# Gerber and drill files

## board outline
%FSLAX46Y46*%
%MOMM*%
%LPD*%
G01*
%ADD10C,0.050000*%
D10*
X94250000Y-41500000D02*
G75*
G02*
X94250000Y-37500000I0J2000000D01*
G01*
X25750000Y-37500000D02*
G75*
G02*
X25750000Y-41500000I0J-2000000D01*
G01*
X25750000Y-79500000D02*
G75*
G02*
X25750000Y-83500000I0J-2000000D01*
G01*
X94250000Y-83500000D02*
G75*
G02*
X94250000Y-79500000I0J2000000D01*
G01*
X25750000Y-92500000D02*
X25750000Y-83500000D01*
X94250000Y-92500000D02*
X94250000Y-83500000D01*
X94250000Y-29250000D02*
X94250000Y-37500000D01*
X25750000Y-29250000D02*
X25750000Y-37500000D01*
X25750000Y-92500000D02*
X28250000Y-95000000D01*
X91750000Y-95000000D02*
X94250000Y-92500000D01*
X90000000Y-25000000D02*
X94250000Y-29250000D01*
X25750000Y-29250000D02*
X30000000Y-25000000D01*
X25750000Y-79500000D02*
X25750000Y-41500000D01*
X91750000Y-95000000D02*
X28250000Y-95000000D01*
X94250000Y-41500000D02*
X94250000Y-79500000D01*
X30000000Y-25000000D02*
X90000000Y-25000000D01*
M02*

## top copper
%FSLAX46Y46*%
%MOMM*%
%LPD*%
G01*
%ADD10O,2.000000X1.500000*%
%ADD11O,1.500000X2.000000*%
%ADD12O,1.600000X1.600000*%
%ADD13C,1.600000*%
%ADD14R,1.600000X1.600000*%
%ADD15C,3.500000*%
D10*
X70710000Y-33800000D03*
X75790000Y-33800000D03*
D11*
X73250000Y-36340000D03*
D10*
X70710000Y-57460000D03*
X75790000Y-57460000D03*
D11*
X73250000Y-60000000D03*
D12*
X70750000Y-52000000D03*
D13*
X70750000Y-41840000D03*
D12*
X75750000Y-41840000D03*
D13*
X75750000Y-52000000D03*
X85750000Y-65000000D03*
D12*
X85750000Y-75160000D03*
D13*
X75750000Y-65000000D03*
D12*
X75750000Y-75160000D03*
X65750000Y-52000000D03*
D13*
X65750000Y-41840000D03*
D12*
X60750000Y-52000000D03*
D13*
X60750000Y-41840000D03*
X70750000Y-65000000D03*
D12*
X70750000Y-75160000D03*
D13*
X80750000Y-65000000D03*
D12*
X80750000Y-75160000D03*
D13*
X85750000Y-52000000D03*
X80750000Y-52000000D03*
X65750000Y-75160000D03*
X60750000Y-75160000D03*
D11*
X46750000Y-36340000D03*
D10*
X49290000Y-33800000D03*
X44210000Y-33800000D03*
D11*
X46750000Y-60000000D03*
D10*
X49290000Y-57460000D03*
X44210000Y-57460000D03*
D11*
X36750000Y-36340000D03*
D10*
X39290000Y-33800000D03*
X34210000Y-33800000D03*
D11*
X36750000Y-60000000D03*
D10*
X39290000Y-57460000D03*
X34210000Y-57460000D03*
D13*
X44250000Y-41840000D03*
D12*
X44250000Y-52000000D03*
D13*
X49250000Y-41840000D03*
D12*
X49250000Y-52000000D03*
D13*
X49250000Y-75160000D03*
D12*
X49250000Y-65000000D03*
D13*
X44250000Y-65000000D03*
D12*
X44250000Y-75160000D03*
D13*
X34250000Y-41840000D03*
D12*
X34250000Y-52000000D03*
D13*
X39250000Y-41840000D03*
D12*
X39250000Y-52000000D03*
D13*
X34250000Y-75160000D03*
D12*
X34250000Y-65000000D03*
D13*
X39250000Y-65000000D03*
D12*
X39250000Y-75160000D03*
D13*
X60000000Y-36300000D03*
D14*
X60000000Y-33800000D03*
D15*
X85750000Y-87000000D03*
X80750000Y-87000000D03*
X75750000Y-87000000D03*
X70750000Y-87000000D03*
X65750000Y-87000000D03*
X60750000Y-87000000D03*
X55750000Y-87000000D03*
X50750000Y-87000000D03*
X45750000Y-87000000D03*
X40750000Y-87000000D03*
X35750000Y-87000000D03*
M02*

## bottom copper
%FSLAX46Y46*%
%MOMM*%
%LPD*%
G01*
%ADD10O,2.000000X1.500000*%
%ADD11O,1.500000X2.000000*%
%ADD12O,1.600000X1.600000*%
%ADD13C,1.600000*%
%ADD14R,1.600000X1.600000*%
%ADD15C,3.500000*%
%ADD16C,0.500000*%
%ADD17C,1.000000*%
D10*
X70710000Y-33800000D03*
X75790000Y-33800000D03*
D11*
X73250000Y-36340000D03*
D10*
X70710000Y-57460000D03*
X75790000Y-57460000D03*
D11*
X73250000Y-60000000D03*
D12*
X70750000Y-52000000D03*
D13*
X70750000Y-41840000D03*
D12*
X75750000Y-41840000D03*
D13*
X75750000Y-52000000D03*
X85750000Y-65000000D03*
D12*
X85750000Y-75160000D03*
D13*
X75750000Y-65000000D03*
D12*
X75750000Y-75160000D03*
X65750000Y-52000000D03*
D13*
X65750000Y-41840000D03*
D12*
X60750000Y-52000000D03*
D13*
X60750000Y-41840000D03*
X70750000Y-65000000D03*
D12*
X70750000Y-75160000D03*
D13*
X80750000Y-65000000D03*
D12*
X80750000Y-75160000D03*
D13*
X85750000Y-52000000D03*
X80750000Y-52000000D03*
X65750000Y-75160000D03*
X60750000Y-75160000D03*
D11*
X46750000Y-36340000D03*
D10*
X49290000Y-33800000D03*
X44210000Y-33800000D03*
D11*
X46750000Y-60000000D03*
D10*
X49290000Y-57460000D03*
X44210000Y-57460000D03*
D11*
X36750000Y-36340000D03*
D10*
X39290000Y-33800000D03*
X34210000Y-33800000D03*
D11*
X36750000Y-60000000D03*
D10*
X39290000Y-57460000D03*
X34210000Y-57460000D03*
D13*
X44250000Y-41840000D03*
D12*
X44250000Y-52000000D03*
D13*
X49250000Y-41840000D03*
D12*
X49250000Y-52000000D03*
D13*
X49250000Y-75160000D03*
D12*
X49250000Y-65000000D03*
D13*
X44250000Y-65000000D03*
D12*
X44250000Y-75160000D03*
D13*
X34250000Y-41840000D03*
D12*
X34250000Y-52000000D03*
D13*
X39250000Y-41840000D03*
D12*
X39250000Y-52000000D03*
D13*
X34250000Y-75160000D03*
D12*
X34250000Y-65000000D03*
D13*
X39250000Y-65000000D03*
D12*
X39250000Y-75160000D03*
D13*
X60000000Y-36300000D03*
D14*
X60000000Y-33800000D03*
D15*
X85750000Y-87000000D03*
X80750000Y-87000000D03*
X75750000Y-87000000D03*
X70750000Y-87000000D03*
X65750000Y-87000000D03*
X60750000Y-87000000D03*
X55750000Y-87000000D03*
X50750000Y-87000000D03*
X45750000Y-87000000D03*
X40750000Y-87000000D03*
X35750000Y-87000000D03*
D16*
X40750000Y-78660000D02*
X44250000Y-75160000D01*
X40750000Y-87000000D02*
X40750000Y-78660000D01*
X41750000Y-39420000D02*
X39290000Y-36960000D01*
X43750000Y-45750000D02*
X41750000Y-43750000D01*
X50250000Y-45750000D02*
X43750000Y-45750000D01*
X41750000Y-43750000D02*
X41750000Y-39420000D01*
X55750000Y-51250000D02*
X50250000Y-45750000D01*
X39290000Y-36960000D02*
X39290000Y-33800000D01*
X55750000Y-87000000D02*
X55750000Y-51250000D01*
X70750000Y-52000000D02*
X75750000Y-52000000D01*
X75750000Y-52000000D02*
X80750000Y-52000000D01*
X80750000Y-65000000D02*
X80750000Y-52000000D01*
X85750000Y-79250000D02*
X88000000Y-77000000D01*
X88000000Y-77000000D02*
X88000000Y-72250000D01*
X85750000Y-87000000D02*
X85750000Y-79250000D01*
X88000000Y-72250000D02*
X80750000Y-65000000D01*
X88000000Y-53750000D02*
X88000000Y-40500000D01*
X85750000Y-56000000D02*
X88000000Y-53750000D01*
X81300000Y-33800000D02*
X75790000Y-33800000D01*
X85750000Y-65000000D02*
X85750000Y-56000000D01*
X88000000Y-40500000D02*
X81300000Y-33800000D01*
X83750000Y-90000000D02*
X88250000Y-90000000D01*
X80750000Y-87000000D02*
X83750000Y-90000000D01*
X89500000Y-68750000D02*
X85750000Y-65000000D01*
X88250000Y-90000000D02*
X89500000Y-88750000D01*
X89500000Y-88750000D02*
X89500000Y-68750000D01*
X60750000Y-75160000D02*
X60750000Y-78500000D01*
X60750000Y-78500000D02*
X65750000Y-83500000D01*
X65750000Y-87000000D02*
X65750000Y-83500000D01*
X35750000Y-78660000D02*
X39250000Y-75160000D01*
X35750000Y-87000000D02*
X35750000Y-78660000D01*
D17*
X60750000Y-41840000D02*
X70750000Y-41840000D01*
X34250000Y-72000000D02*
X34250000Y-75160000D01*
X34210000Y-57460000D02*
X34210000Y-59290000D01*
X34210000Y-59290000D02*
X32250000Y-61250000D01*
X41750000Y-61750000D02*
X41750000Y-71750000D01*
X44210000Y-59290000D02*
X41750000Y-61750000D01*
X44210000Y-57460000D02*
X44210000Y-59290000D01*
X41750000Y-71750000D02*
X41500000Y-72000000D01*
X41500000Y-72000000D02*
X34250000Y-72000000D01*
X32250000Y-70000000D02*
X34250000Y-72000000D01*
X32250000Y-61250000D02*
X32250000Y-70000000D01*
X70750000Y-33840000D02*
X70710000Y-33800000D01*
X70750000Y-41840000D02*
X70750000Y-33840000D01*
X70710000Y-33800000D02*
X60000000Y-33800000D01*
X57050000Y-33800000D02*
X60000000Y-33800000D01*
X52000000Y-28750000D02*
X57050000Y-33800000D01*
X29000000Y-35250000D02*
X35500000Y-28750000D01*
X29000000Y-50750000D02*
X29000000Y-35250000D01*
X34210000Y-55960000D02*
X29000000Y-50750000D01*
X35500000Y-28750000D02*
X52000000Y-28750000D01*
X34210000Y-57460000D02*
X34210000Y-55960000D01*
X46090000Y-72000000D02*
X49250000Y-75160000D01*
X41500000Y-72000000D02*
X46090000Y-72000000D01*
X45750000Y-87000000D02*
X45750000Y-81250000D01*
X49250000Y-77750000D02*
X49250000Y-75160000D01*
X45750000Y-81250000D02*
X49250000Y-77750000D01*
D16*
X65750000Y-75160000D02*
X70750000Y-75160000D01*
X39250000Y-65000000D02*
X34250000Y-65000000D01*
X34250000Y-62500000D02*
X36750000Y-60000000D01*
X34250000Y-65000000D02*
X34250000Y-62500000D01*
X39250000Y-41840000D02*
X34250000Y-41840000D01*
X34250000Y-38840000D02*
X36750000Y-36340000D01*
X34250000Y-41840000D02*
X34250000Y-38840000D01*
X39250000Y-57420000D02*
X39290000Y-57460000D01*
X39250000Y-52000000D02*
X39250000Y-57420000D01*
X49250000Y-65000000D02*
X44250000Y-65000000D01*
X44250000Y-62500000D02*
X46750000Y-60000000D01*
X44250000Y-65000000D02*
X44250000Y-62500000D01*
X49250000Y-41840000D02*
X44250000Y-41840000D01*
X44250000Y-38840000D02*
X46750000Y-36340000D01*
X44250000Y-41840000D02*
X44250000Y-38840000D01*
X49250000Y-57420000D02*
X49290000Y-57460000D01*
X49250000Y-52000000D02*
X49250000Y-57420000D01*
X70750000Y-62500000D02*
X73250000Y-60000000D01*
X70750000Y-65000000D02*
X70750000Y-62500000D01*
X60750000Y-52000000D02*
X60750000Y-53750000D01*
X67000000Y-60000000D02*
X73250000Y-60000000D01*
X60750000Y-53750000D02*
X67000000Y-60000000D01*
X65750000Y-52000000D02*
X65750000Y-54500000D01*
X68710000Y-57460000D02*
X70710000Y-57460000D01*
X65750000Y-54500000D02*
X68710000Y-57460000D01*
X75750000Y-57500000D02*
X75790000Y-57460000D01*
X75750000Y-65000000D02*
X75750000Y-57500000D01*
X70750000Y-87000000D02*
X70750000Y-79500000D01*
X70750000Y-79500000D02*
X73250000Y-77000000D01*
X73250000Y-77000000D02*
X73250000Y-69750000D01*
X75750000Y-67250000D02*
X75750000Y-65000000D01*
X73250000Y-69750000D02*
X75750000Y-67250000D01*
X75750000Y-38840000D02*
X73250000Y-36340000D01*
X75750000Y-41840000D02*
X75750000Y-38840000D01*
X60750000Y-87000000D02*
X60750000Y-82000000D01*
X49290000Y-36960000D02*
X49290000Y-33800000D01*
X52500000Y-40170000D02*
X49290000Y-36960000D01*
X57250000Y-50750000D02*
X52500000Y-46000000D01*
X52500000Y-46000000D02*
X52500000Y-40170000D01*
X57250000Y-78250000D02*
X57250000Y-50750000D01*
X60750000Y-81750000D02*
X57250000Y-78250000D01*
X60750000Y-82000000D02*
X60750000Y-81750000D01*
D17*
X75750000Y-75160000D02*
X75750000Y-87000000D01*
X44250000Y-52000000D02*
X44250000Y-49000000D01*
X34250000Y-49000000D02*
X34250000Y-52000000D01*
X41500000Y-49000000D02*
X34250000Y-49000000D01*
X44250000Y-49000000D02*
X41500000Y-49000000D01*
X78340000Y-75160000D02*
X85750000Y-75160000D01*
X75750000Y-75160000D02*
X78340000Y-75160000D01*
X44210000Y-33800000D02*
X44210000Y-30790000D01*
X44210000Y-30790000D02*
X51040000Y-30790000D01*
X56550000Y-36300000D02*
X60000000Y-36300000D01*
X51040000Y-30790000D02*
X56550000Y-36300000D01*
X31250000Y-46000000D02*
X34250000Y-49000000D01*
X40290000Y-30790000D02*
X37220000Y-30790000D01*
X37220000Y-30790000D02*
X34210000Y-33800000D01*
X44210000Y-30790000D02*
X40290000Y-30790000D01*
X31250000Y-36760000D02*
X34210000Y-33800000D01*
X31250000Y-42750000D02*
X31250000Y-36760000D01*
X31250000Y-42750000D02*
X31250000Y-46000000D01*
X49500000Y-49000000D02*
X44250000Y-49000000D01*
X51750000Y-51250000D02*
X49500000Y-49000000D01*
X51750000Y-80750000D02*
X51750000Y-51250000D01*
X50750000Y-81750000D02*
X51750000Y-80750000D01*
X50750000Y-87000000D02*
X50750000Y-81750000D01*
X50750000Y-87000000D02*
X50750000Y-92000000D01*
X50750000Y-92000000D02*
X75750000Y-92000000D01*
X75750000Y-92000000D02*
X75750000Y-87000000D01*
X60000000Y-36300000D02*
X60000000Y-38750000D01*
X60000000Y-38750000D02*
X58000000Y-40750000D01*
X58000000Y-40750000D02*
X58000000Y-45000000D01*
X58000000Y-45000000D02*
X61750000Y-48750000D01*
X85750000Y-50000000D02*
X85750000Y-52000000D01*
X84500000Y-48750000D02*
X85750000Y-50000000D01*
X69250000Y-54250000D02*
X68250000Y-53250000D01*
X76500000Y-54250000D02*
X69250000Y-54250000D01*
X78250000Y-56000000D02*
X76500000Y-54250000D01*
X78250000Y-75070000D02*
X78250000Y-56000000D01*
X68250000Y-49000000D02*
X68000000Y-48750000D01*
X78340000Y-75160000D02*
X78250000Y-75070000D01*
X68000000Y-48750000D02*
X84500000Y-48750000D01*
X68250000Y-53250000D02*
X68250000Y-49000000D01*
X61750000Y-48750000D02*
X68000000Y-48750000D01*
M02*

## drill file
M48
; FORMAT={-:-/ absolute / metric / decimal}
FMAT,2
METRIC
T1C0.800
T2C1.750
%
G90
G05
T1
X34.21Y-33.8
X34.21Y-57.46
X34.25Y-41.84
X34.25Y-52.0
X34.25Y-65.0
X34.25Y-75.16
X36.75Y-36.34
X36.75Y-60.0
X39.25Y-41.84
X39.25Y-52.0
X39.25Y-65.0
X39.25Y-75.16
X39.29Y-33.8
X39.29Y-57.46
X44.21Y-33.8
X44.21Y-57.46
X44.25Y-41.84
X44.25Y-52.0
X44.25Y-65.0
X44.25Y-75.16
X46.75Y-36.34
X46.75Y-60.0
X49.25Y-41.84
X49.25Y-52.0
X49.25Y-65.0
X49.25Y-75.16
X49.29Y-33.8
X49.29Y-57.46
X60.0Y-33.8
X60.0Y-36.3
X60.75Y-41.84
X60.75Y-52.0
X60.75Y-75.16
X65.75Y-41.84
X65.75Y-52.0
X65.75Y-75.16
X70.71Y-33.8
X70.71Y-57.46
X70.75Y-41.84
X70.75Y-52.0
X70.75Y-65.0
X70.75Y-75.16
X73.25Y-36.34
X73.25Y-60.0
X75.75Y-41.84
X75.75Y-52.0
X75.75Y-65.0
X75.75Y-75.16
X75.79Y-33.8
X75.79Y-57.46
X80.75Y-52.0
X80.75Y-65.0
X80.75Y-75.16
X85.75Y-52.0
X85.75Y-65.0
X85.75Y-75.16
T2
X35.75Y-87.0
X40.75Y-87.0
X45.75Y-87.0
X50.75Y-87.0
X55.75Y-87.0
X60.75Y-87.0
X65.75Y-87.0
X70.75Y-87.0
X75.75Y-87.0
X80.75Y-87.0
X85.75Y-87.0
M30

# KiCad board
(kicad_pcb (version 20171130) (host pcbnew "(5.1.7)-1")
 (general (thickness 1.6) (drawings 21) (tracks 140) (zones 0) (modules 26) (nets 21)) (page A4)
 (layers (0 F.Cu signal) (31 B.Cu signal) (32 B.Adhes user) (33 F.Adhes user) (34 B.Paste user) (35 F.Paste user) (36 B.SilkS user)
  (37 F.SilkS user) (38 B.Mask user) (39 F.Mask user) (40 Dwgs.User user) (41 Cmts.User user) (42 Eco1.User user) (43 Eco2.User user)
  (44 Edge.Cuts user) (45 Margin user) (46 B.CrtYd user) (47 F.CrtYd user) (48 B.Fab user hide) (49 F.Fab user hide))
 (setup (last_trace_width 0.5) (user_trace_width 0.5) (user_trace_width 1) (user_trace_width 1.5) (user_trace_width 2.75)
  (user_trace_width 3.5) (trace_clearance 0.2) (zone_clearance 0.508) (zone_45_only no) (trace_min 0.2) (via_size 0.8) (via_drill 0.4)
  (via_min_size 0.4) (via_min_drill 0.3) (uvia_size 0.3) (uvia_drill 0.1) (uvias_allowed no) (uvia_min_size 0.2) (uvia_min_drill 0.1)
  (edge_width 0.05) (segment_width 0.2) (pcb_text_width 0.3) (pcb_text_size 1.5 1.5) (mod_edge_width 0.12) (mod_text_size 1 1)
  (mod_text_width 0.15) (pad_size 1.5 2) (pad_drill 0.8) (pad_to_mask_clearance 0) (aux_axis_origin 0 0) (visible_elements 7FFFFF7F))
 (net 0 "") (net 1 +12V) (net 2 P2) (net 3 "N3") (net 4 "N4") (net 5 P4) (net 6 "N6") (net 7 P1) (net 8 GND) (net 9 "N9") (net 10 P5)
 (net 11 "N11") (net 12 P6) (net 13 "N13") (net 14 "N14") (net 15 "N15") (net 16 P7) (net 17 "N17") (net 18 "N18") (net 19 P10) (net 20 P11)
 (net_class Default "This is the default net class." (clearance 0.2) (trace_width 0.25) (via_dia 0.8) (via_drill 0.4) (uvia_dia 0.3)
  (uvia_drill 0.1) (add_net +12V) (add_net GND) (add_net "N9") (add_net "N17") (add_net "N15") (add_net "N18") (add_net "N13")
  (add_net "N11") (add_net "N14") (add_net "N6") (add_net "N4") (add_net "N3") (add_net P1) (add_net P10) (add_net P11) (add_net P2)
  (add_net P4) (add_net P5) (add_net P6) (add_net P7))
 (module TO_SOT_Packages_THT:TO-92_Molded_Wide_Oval (layer F.Cu) (at 75.79 33.8 180)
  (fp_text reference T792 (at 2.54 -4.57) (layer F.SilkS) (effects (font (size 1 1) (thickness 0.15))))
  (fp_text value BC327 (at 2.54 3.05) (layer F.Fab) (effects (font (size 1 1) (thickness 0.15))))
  (pad 3 thru_hole oval (at 5.08 0 270) (size 1.5 2) (drill 0.8) (layers *.Cu *.Mask) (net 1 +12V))
  (pad 1 thru_hole oval (at 0 0 270) (size 1.5 2) (drill 0.8) (layers *.Cu *.Mask) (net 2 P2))
  (pad 2 thru_hole oval (at 2.54 -2.54 270) (size 2 1.5) (drill 0.8) (layers *.Cu *.Mask) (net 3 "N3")))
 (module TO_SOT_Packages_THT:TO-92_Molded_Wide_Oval (layer F.Cu) (at 75.79 57.46 180)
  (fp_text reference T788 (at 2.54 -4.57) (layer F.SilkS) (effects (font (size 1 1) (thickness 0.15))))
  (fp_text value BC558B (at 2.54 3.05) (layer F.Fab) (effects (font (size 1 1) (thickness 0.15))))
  (pad 3 thru_hole oval (at 5.08 0 270) (size 1.5 2) (drill 0.8) (layers *.Cu *.Mask) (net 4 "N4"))
  (pad 1 thru_hole oval (at 0 0 270) (size 1.5 2) (drill 0.8) (layers *.Cu *.Mask) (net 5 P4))
  (pad 2 thru_hole oval (at 2.54 -2.54 270) (size 2 1.5) (drill 0.8) (layers *.Cu *.Mask) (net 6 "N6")))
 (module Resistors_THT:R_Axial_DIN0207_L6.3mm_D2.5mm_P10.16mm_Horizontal (layer F.Cu) (at 70.75 41.84 270)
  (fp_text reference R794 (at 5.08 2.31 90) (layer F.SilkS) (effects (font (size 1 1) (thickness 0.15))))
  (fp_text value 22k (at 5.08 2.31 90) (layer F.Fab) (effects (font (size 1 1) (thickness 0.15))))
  (pad 2 thru_hole oval (at 10.16 0 270) (size 1.6 1.6) (drill 0.8) (layers *.Cu *.Mask) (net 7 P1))
  (pad 1 thru_hole circle (at 0 0 270) (size 1.6 1.6) (drill 0.8) (layers *.Cu *.Mask) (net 1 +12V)))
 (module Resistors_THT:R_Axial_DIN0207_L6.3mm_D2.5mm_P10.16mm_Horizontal (layer F.Cu) (at 75.75 52 90)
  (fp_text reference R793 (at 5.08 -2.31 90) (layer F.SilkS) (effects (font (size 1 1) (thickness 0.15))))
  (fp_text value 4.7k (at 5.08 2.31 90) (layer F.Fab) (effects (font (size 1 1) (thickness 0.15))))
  (pad 2 thru_hole oval (at 10.16 0 90) (size 1.6 1.6) (drill 0.8) (layers *.Cu *.Mask) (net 3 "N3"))
  (pad 1 thru_hole circle (at 0 0 90) (size 1.6 1.6) (drill 0.8) (layers *.Cu *.Mask) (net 7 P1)))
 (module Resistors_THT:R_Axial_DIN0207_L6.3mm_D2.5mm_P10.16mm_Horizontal (layer F.Cu) (at 85.75 65 270)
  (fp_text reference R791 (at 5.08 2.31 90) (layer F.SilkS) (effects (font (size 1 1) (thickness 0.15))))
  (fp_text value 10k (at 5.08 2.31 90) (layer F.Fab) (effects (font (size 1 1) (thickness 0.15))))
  (pad 1 thru_hole circle (at 0 0 270) (size 1.6 1.6) (drill 0.8) (layers *.Cu *.Mask) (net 2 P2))
  (pad 2 thru_hole oval (at 10.16 0 270) (size 1.6 1.6) (drill 0.8) (layers *.Cu *.Mask) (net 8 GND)))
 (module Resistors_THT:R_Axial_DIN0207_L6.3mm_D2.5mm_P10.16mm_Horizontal (layer F.Cu) (at 75.75 65 270)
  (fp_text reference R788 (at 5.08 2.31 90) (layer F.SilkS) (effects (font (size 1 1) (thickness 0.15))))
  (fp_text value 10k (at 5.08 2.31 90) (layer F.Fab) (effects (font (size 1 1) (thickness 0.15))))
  (pad 1 thru_hole circle (at 0 0 270) (size 1.6 1.6) (drill 0.8) (layers *.Cu *.Mask) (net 5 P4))
  (pad 2 thru_hole oval (at 10.16 0 270) (size 1.6 1.6) (drill 0.8) (layers *.Cu *.Mask) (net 8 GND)))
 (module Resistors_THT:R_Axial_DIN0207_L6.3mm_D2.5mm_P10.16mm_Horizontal (layer F.Cu) (at 65.75 41.84 270)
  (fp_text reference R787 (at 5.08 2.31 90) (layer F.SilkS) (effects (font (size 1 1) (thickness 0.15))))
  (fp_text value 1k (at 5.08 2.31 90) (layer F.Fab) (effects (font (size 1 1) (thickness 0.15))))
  (pad 2 thru_hole oval (at 10.16 0 270) (size 1.6 1.6) (drill 0.8) (layers *.Cu *.Mask) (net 4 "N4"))
  (pad 1 thru_hole circle (at 0 0 270) (size 1.6 1.6) (drill 0.8) (layers *.Cu *.Mask) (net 1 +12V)))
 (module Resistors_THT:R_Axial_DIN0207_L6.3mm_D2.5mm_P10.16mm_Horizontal (layer F.Cu) (at 60.75 41.84 270)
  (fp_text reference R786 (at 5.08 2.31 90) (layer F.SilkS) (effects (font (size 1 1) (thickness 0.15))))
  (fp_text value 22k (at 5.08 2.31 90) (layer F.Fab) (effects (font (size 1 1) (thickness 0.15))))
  (pad 2 thru_hole oval (at 10.16 0 270) (size 1.6 1.6) (drill 0.8) (layers *.Cu *.Mask) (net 6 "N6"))
  (pad 1 thru_hole circle (at 0 0 270) (size 1.6 1.6) (drill 0.8) (layers *.Cu *.Mask) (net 1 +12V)))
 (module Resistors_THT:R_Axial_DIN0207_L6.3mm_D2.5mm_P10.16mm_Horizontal (layer F.Cu) (at 70.75 65 270)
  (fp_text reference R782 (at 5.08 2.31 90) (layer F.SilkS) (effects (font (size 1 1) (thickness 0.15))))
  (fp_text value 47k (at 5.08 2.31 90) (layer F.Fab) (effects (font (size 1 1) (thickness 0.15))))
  (pad 1 thru_hole circle (at 0 0 270) (size 1.6 1.6) (drill 0.8) (layers *.Cu *.Mask) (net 6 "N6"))
  (pad 2 thru_hole oval (at 10.16 0 270) (size 1.6 1.6) (drill 0.8) (layers *.Cu *.Mask) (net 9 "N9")))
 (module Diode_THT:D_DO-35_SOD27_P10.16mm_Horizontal (layer F.Cu) (at 80.75 65 270)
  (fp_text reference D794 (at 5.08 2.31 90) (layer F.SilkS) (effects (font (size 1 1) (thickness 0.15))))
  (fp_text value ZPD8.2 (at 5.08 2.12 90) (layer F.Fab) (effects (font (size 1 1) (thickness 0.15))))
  (pad 1 thru_hole circle (at 0 0 270) (size 1.6 1.6) (drill 0.8) (layers *.Cu *.Mask) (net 7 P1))
  (pad 2 thru_hole oval (at 10.16 0 270) (size 1.6 1.6) (drill 0.8) (layers *.Cu *.Mask) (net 8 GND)))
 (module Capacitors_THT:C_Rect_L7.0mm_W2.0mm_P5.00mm (layer F.Cu) (at 80.75 52)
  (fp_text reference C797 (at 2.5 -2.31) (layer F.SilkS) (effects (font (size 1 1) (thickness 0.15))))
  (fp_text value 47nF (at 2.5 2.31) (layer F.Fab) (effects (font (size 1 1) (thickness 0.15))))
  (pad 2 thru_hole circle (at 5 0) (size 1.6 1.6) (drill 0.8) (layers *.Cu *.Mask) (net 8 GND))
  (pad 1 thru_hole circle (at 0 0) (size 1.6 1.6) (drill 0.8) (layers *.Cu *.Mask) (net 7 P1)))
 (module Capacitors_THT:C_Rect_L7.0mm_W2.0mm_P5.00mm (layer F.Cu) (at 65.75 75.16 180)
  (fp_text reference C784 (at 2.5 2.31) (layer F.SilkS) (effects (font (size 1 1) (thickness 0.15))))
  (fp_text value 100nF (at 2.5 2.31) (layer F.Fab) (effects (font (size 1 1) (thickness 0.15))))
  (pad 1 thru_hole circle (at 0 0 180) (size 1.6 1.6) (drill 0.8) (layers *.Cu *.Mask) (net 9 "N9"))
  (pad 2 thru_hole circle (at 5 0 180) (size 1.6 1.6) (drill 0.8) (layers *.Cu *.Mask) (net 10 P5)))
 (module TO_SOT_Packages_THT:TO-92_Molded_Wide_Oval (layer F.Cu) (at 49.29 33.8 180)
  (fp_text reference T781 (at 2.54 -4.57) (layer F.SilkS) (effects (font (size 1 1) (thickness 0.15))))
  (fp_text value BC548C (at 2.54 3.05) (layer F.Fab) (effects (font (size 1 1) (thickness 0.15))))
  (pad 2 thru_hole oval (at 2.54 -2.54 270) (size 2 1.5) (drill 0.8) (layers *.Cu *.Mask) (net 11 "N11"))
  (pad 1 thru_hole oval (at 0 0 270) (size 1.5 2) (drill 0.8) (layers *.Cu *.Mask) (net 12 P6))
  (pad 3 thru_hole oval (at 5.08 0 270) (size 1.5 2) (drill 0.8) (layers *.Cu *.Mask) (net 8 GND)))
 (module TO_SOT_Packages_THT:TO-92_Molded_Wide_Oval (layer F.Cu) (at 49.29 57.46 180)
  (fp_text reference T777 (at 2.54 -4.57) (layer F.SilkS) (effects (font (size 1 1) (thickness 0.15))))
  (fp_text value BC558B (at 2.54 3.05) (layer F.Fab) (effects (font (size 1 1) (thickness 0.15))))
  (pad 2 thru_hole oval (at 2.54 -2.54 270) (size 2 1.5) (drill 0.8) (layers *.Cu *.Mask) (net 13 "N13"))
  (pad 1 thru_hole oval (at 0 0 270) (size 1.5 2) (drill 0.8) (layers *.Cu *.Mask) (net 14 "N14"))
  (pad 3 thru_hole oval (at 5.08 0 270) (size 1.5 2) (drill 0.8) (layers *.Cu *.Mask) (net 1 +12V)))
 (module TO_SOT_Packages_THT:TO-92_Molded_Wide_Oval (layer F.Cu) (at 39.29 33.8 180)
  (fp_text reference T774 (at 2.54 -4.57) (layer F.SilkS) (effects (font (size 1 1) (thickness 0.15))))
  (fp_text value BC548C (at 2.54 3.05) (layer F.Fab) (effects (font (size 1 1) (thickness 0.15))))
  (pad 2 thru_hole oval (at 2.54 -2.54 270) (size 2 1.5) (drill 0.8) (layers *.Cu *.Mask) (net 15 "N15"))
  (pad 1 thru_hole oval (at 0 0 270) (size 1.5 2) (drill 0.8) (layers *.Cu *.Mask) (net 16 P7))
  (pad 3 thru_hole oval (at 5.08 0 270) (size 1.5 2) (drill 0.8) (layers *.Cu *.Mask) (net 8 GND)))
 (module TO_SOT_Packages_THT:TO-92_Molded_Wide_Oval (layer F.Cu) (at 39.29 57.46 180)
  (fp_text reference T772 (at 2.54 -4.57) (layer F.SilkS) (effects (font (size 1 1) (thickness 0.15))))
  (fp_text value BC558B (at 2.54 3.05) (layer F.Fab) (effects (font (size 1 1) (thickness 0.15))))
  (pad 2 thru_hole oval (at 2.54 -2.54 270) (size 2 1.5) (drill 0.8) (layers *.Cu *.Mask) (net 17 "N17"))
  (pad 1 thru_hole oval (at 0 0 270) (size 1.5 2) (drill 0.8) (layers *.Cu *.Mask) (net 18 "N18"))
  (pad 3 thru_hole oval (at 5.08 0 270) (size 1.5 2) (drill 0.8) (layers *.Cu *.Mask) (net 1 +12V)))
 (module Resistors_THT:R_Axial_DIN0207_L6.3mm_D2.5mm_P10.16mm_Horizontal (layer F.Cu) (at 44.25 41.84 270)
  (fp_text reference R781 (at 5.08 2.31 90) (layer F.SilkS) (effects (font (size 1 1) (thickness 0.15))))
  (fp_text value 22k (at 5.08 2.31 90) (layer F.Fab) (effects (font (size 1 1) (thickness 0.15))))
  (pad 1 thru_hole circle (at 0 0 270) (size 1.6 1.6) (drill 0.8) (layers *.Cu *.Mask) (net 11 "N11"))
  (pad 2 thru_hole oval (at 10.16 0 270) (size 1.6 1.6) (drill 0.8) (layers *.Cu *.Mask) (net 8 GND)))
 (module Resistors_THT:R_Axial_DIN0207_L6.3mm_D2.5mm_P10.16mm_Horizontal (layer F.Cu) (at 49.25 41.84 270)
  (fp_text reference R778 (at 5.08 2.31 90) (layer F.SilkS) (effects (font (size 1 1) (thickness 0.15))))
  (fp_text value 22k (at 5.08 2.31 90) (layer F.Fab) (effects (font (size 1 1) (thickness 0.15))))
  (pad 1 thru_hole circle (at 0 0 270) (size 1.6 1.6) (drill 0.8) (layers *.Cu *.Mask) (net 11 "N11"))
  (pad 2 thru_hole oval (at 10.16 0 270) (size 1.6 1.6) (drill 0.8) (layers *.Cu *.Mask) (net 14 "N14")))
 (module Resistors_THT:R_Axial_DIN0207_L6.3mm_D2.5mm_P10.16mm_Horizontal (layer F.Cu) (at 49.25 75.16 90)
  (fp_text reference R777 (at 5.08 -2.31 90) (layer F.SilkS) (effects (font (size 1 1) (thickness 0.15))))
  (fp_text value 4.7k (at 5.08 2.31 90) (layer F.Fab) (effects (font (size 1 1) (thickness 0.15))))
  (pad 1 thru_hole circle (at 0 0 90) (size 1.6 1.6) (drill 0.8) (layers *.Cu *.Mask) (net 1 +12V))
  (pad 2 thru_hole oval (at 10.16 0 90) (size 1.6 1.6) (drill 0.8) (layers *.Cu *.Mask) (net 13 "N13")))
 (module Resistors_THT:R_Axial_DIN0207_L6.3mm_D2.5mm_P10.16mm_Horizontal (layer F.Cu) (at 44.25 65 270)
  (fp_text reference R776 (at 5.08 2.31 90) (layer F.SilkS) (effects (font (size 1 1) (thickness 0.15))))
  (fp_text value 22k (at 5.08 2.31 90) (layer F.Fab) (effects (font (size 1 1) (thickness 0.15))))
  (pad 1 thru_hole circle (at 0 0 270) (size 1.6 1.6) (drill 0.8) (layers *.Cu *.Mask) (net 13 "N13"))
  (pad 2 thru_hole oval (at 10.16 0 270) (size 1.6 1.6) (drill 0.8) (layers *.Cu *.Mask) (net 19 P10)))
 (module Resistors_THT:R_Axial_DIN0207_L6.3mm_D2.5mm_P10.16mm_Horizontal (layer F.Cu) (at 34.25 41.84 270)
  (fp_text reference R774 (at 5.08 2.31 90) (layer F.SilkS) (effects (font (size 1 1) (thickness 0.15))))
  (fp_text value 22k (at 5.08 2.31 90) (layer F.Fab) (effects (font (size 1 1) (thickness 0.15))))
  (pad 1 thru_hole circle (at 0 0 270) (size 1.6 1.6) (drill 0.8) (layers *.Cu *.Mask) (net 15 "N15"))
  (pad 2 thru_hole oval (at 10.16 0 270) (size 1.6 1.6) (drill 0.8) (layers *.Cu *.Mask) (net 8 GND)))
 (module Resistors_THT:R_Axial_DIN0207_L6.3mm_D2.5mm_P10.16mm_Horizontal (layer F.Cu) (at 39.25 41.84 270)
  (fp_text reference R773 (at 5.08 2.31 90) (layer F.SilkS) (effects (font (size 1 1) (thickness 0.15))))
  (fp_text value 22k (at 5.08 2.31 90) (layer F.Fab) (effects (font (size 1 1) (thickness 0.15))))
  (pad 1 thru_hole circle (at 0 0 270) (size 1.6 1.6) (drill 0.8) (layers *.Cu *.Mask) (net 15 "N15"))
  (pad 2 thru_hole oval (at 10.16 0 270) (size 1.6 1.6) (drill 0.8) (layers *.Cu *.Mask) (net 18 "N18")))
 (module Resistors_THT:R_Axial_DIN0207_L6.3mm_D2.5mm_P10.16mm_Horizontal (layer F.Cu) (at 34.25 75.16 90)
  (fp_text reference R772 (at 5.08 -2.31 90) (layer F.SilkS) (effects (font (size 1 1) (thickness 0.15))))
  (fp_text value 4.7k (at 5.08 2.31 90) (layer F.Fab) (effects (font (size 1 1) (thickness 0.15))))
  (pad 1 thru_hole circle (at 0 0 90) (size 1.6 1.6) (drill 0.8) (layers *.Cu *.Mask) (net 1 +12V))
  (pad 2 thru_hole oval (at 10.16 0 90) (size 1.6 1.6) (drill 0.8) (layers *.Cu *.Mask) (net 17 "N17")))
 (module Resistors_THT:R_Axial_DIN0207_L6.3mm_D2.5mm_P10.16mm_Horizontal (layer F.Cu) (at 39.25 65 270)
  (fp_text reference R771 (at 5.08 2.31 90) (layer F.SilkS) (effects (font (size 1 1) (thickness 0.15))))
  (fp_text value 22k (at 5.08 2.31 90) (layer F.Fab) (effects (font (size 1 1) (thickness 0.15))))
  (pad 1 thru_hole circle (at 0 0 270) (size 1.6 1.6) (drill 0.8) (layers *.Cu *.Mask) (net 17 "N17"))
  (pad 2 thru_hole oval (at 10.16 0 270) (size 1.6 1.6) (drill 0.8) (layers *.Cu *.Mask) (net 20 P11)))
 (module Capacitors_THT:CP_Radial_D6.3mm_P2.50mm (layer F.Cu) (at 60 33.8 270)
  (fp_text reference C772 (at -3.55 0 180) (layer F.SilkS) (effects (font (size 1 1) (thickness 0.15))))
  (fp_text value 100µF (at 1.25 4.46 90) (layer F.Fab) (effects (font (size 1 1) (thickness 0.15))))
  (pad 2 thru_hole circle (at 2.5 0 270) (size 1.6 1.6) (drill 0.8) (layers *.Cu *.Mask) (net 8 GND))
  (pad 1 thru_hole rect (at 0 0 270) (size 1.6 1.6) (drill 0.8) (layers *.Cu *.Mask) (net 1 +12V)))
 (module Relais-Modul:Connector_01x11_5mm (layer F.Cu) (at 85.75 87)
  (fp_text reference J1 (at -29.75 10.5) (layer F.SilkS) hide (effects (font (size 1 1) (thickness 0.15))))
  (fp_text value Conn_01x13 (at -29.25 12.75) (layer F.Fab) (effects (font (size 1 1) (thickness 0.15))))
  (pad 1 thru_hole circle (at 0 0 180) (size 3.5 3.5) (drill 1.75) (layers B.Cu B.Mask) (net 7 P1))
  (pad 2 thru_hole circle (at -5 0 180) (size 3.5 3.5) (drill 1.75) (layers B.Cu B.Mask) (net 2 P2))
  (pad 3 thru_hole circle (at -10 0 180) (size 3.5 3.5) (drill 1.75) (layers B.Cu B.Mask) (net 8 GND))
  (pad 4 thru_hole circle (at -15 0 180) (size 3.5 3.5) (drill 1.75) (layers B.Cu B.Mask) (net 5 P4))
  (pad 5 thru_hole circle (at -20 0 180) (size 3.5 3.5) (drill 1.75) (layers B.Cu B.Mask) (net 10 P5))
  (pad 6 thru_hole circle (at -25 0 180) (size 3.5 3.5) (drill 1.75) (layers B.Cu B.Mask) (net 12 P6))
  (pad 7 thru_hole circle (at -30 0 180) (size 3.5 3.5) (drill 1.75) (layers B.Cu B.Mask) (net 16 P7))
  (pad 8 thru_hole circle (at -35 0 180) (size 3.5 3.5) (drill 1.75) (layers B.Cu B.Mask) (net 8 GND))
  (pad 9 thru_hole circle (at -40 0 180) (size 3.5 3.5) (drill 1.75) (layers B.Cu B.Mask) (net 1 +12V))
  (pad 10 thru_hole circle (at -45 0 180) (size 3.5 3.5) (drill 1.75) (layers B.Cu B.Mask) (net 19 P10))
  (pad 11 thru_hole circle (at -50 0 180) (size 3.5 3.5) (drill 1.75) (layers B.Cu B.Mask) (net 20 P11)))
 (gr_arc (start 94.25 39.5) (end 94.25 37.5) (angle -180) (layer Edge.Cuts) (width 0.05))
 (gr_arc (start 25.75 39.5) (end 25.75 41.5) (angle -180) (layer Edge.Cuts) (width 0.05))
 (gr_arc (start 25.75 81.5) (end 25.75 83.5) (angle -180) (layer Edge.Cuts) (width 0.05))
 (gr_arc (start 94.25 81.5) (end 94.25 79.5) (angle -180) (layer Edge.Cuts) (width 0.05))
 (gr_line (start 25.75 92.5) (end 25.75 83.5) (layer Edge.Cuts) (width 0.05))
 (gr_line (start 94.25 92.5) (end 94.25 83.5) (layer Edge.Cuts) (width 0.05))
 (gr_line (start 94.25 29.25) (end 94.25 37.5) (layer Edge.Cuts) (width 0.05))
 (gr_line (start 25.75 29.25) (end 25.75 37.5) (layer Edge.Cuts) (width 0.05))
 (gr_line (start 25.75 92.5) (end 28.25 95) (layer Edge.Cuts) (width 0.05))
 (gr_line (start 91.75 95) (end 94.25 92.5) (layer Edge.Cuts) (width 0.05))
 (gr_line (start 90 25) (end 94.25 29.25) (layer Edge.Cuts) (width 0.05))
 (gr_line (start 25.75 29.25) (end 30 25) (layer Edge.Cuts) (width 0.05))
 (gr_line (start 25.75 79.5) (end 25.75 41.5) (layer Edge.Cuts) (width 0.05))
 (gr_line (start 91.75 95) (end 28.25 95) (layer Edge.Cuts) (width 0.05))
 (gr_line (start 94.25 41.5) (end 94.25 79.5) (layer Edge.Cuts) (width 0.05))
 (gr_line (start 30 25) (end 90 25) (layer Edge.Cuts) (width 0.05))
 (segment (start 40.75 78.66) (end 44.25 75.16) (width 0.5) (layer B.Cu) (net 19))
 (segment (start 40.75 87) (end 40.75 78.66) (width 0.5) (layer B.Cu) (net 19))
 (segment (start 41.75 39.42) (end 39.29 36.96) (width 0.5) (layer B.Cu) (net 16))
 (segment (start 43.75 45.75) (end 41.75 43.75) (width 0.5) (layer B.Cu) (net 16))
 (segment (start 50.25 45.75) (end 43.75 45.75) (width 0.5) (layer B.Cu) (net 16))
 (segment (start 41.75 43.75) (end 41.75 39.42) (width 0.5) (layer B.Cu) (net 16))
 (segment (start 55.75 51.25) (end 50.25 45.75) (width 0.5) (layer B.Cu) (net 16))
 (segment (start 39.29 36.96) (end 39.29 33.8) (width 0.5) (layer B.Cu) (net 16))
 (segment (start 55.75 87) (end 55.75 51.25) (width 0.5) (layer B.Cu) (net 16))
 (segment (start 70.75 52) (end 75.75 52) (width 0.5) (layer B.Cu) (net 7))
 (segment (start 75.75 52) (end 80.75 52) (width 0.5) (layer B.Cu) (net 7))
 (segment (start 80.75 65) (end 80.75 52) (width 0.5) (layer B.Cu) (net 7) (status 1000000))
 (segment (start 85.75 79.25) (end 88 77) (width 0.5) (layer B.Cu) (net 7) (status 1000000))
 (segment (start 88 77) (end 88 72.25) (width 0.5) (layer B.Cu) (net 7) (status 1000000))
 (segment (start 85.75 87) (end 85.75 79.25) (width 0.5) (layer B.Cu) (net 7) (status 1000000))
 (segment (start 88 72.25) (end 80.75 65) (width 0.5) (layer B.Cu) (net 7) (status 1000000))
 (segment (start 88 53.75) (end 88 40.5) (width 0.5) (layer B.Cu) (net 2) (status 1000000))
 (segment (start 85.75 56) (end 88 53.75) (width 0.5) (layer B.Cu) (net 2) (status 1000000))
 (segment (start 81.3 33.8) (end 75.79 33.8) (width 0.5) (layer B.Cu) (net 2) (status 1000000))
 (segment (start 85.75 65) (end 85.75 56) (width 0.5) (layer B.Cu) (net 2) (status 1000000))
 (segment (start 88 40.5) (end 81.3 33.8) (width 0.5) (layer B.Cu) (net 2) (status 1000000))
 (segment (start 83.75 90) (end 88.25 90) (width 0.5) (layer B.Cu) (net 2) (status 1000000))
 (segment (start 80.75 87) (end 83.75 90) (width 0.5) (layer B.Cu) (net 2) (status 1000000))
 (segment (start 89.5 68.75) (end 85.75 65) (width 0.5) (layer B.Cu) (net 2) (status 1000000))
 (segment (start 88.25 90) (end 89.5 88.75) (width 0.5) (layer B.Cu) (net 2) (status 1000000))
 (segment (start 89.5 88.75) (end 89.5 68.75) (width 0.5) (layer B.Cu) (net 2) (status 1000000))
 (segment (start 60.75 75.16) (end 60.75 78.5) (width 0.5) (layer B.Cu) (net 10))
 (segment (start 60.75 78.5) (end 65.75 83.5) (width 0.5) (layer B.Cu) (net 10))
 (segment (start 65.75 87) (end 65.75 83.5) (width 0.5) (layer B.Cu) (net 10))
 (segment (start 35.75 78.66) (end 39.25 75.16) (width 0.5) (layer B.Cu) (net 20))
 (segment (start 35.75 87) (end 35.75 78.66) (width 0.5) (layer B.Cu) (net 20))
 (segment (start 60.75 41.84) (end 70.75 41.84) (width 1) (layer B.Cu) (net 1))
 (segment (start 34.25 72) (end 34.25 75.16) (width 1) (layer B.Cu) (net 1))
 (segment (start 34.21 57.46) (end 34.21 59.29) (width 1) (layer B.Cu) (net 1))
 (segment (start 34.21 59.29) (end 32.25 61.25) (width 1) (layer B.Cu) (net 1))
 (segment (start 41.75 61.75) (end 41.75 71.75) (width 1) (layer B.Cu) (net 1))
 (segment (start 44.21 59.29) (end 41.75 61.75) (width 1) (layer B.Cu) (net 1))
 (segment (start 44.21 57.46) (end 44.21 59.29) (width 1) (layer B.Cu) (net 1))
 (segment (start 41.75 71.75) (end 41.5 72) (width 1) (layer B.Cu) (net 1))
 (segment (start 41.5 72) (end 34.25 72) (width 1) (layer B.Cu) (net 1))
 (segment (start 32.25 70) (end 34.25 72) (width 1) (layer B.Cu) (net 1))
 (segment (start 32.25 61.25) (end 32.25 70) (width 1) (layer B.Cu) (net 1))
 (segment (start 70.75 33.84) (end 70.71 33.8) (width 1) (layer B.Cu) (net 1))
 (segment (start 70.75 41.84) (end 70.75 33.84) (width 1) (layer B.Cu) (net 1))
 (segment (start 70.71 33.8) (end 60 33.8) (width 1) (layer B.Cu) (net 1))
 (segment (start 57.05 33.8) (end 60 33.8) (width 1) (layer B.Cu) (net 1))
 (segment (start 52 28.75) (end 57.05 33.8) (width 1) (layer B.Cu) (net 1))
 (segment (start 29 35.25) (end 35.5 28.75) (width 1) (layer B.Cu) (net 1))
 (segment (start 29 50.75) (end 29 35.25) (width 1) (layer B.Cu) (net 1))
 (segment (start 34.21 55.96) (end 29 50.75) (width 1) (layer B.Cu) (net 1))
 (segment (start 35.5 28.75) (end 52 28.75) (width 1) (layer B.Cu) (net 1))
 (segment (start 34.21 57.46) (end 34.21 55.96) (width 1) (layer B.Cu) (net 1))
 (segment (start 46.09 72) (end 49.25 75.16) (width 1) (layer B.Cu) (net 1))
 (segment (start 41.5 72) (end 46.09 72) (width 1) (layer B.Cu) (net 1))
 (segment (start 45.75 87) (end 45.75 81.25) (width 1) (layer B.Cu) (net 1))
 (segment (start 49.25 77.75) (end 49.25 75.16) (width 1) (layer B.Cu) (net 1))
 (segment (start 45.75 81.25) (end 49.25 77.75) (width 1) (layer B.Cu) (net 1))
 (segment (start 65.75 75.16) (end 70.75 75.16) (width 0.5) (layer B.Cu) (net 9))
 (segment (start 39.25 65) (end 34.25 65) (width 0.5) (layer B.Cu) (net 17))
 (segment (start 34.25 62.5) (end 36.75 60) (width 0.5) (layer B.Cu) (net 17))
 (segment (start 34.25 65) (end 34.25 62.5) (width 0.5) (layer B.Cu) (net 17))
 (segment (start 39.25 41.84) (end 34.25 41.84) (width 0.5) (layer B.Cu) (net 15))
 (segment (start 34.25 38.84) (end 36.75 36.34) (width 0.5) (layer B.Cu) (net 15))
 (segment (start 34.25 41.84) (end 34.25 38.84) (width 0.5) (layer B.Cu) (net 15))
 (segment (start 39.25 57.42) (end 39.29 57.46) (width 0.5) (layer B.Cu) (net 18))
 (segment (start 39.25 52) (end 39.25 57.42) (width 0.5) (layer B.Cu) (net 18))
 (segment (start 49.25 65) (end 44.25 65) (width 0.5) (layer B.Cu) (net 13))
 (segment (start 44.25 62.5) (end 46.75 60) (width 0.5) (layer B.Cu) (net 13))
 (segment (start 44.25 65) (end 44.25 62.5) (width 0.5) (layer B.Cu) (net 13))
 (segment (start 49.25 41.84) (end 44.25 41.84) (width 0.5) (layer B.Cu) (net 11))
 (segment (start 44.25 38.84) (end 46.75 36.34) (width 0.5) (layer B.Cu) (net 11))
 (segment (start 44.25 41.84) (end 44.25 38.84) (width 0.5) (layer B.Cu) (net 11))
 (segment (start 49.25 57.42) (end 49.29 57.46) (width 0.5) (layer B.Cu) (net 14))
 (segment (start 49.25 52) (end 49.25 57.42) (width 0.5) (layer B.Cu) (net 14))
 (segment (start 70.75 62.5) (end 73.25 60) (width 0.5) (layer B.Cu) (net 6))
 (segment (start 70.75 65) (end 70.75 62.5) (width 0.5) (layer B.Cu) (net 6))
 (segment (start 60.75 52) (end 60.75 53.75) (width 0.5) (layer B.Cu) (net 6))
 (segment (start 67 60) (end 73.25 60) (width 0.5) (layer B.Cu) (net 6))
 (segment (start 60.75 53.75) (end 67 60) (width 0.5) (layer B.Cu) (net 6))
 (segment (start 65.75 52) (end 65.75 54.5) (width 0.5) (layer B.Cu) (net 4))
 (segment (start 68.71 57.46) (end 70.71 57.46) (width 0.5) (layer B.Cu) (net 4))
 (segment (start 65.75 54.5) (end 68.71 57.46) (width 0.5) (layer B.Cu) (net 4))
 (segment (start 75.75 57.5) (end 75.79 57.46) (width 0.5) (layer B.Cu) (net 5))
 (segment (start 75.75 65) (end 75.75 57.5) (width 0.5) (layer B.Cu) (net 5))
 (segment (start 70.75 87) (end 70.75 79.5) (width 0.5) (layer B.Cu) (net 5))
 (segment (start 70.75 79.5) (end 73.25 77) (width 0.5) (layer B.Cu) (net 5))
 (segment (start 73.25 77) (end 73.25 69.75) (width 0.5) (layer B.Cu) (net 5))
 (segment (start 75.75 67.25) (end 75.75 65) (width 0.5) (layer B.Cu) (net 5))
 (segment (start 73.25 69.75) (end 75.75 67.25) (width 0.5) (layer B.Cu) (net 5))
 (segment (start 75.75 38.84) (end 73.25 36.34) (width 0.5) (layer B.Cu) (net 3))
 (segment (start 75.75 41.84) (end 75.75 38.84) (width 0.5) (layer B.Cu) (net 3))
 (segment (start 60.75 87) (end 60.75 82) (width 0.5) (layer B.Cu) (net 12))
 (segment (start 49.29 36.96) (end 49.29 33.8) (width 0.5) (layer B.Cu) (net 12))
 (segment (start 52.5 40.17) (end 49.29 36.96) (width 0.5) (layer B.Cu) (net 12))
 (segment (start 57.25 50.75) (end 52.5 46) (width 0.5) (layer B.Cu) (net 12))
 (segment (start 52.5 46) (end 52.5 40.17) (width 0.5) (layer B.Cu) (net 12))
 (segment (start 57.25 78.25) (end 57.25 50.75) (width 0.5) (layer B.Cu) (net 12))
 (segment (start 60.75 81.75) (end 57.25 78.25) (width 0.5) (layer B.Cu) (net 12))
 (segment (start 60.75 82) (end 60.75 81.75) (width 0.5) (layer B.Cu) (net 12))
 (segment (start 75.75 75.16) (end 75.75 87) (width 1) (layer B.Cu) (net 8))
 (segment (start 44.25 52) (end 44.25 49) (width 1) (layer B.Cu) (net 8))
 (segment (start 34.25 49) (end 34.25 52) (width 1) (layer B.Cu) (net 8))
 (segment (start 41.5 49) (end 34.25 49) (width 1) (layer B.Cu) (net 8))
 (segment (start 44.25 49) (end 41.5 49) (width 1) (layer B.Cu) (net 8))
 (segment (start 78.34 75.16) (end 85.75 75.16) (width 1) (layer B.Cu) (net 8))
 (segment (start 75.75 75.16) (end 78.34 75.16) (width 1) (layer B.Cu) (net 8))
 (segment (start 44.21 33.8) (end 44.21 30.79) (width 1) (layer B.Cu) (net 8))
 (segment (start 44.21 30.79) (end 51.04 30.79) (width 1) (layer B.Cu) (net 8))
 (segment (start 56.55 36.3) (end 60 36.3) (width 1) (layer B.Cu) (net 8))
 (segment (start 51.04 30.79) (end 56.55 36.3) (width 1) (layer B.Cu) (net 8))
 (segment (start 31.25 46) (end 34.25 49) (width 1) (layer B.Cu) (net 8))
 (segment (start 40.29 30.79) (end 37.22 30.79) (width 1) (layer B.Cu) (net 8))
 (segment (start 37.22 30.79) (end 34.21 33.8) (width 1) (layer B.Cu) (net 8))
 (segment (start 44.21 30.79) (end 40.29 30.79) (width 1) (layer B.Cu) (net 8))
 (segment (start 31.25 36.76) (end 34.21 33.8) (width 1) (layer B.Cu) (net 8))
 (segment (start 31.25 42.75) (end 31.25 36.76) (width 1) (layer B.Cu) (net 8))
 (segment (start 31.25 42.75) (end 31.25 46) (width 1) (layer B.Cu) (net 8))
 (segment (start 49.5 49) (end 44.25 49) (width 1) (layer B.Cu) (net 8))
 (segment (start 51.75 51.25) (end 49.5 49) (width 1) (layer B.Cu) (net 8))
 (segment (start 51.75 80.75) (end 51.75 51.25) (width 1) (layer B.Cu) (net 8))
 (segment (start 50.75 81.75) (end 51.75 80.75) (width 1) (layer B.Cu) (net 8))
 (segment (start 50.75 87) (end 50.75 81.75) (width 1) (layer B.Cu) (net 8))
 (segment (start 50.75 87) (end 50.75 92) (width 1) (layer B.Cu) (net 8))
 (segment (start 50.75 92) (end 75.75 92) (width 1) (layer B.Cu) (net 8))
 (segment (start 75.75 92) (end 75.75 87) (width 1) (layer B.Cu) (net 8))
 (segment (start 60 36.3) (end 60 38.75) (width 1) (layer B.Cu) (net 8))
 (segment (start 60 38.75) (end 58 40.75) (width 1) (layer B.Cu) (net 8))
 (segment (start 58 40.75) (end 58 45) (width 1) (layer B.Cu) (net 8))
 (segment (start 58 45) (end 61.75 48.75) (width 1) (layer B.Cu) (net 8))
 (segment (start 85.75 50) (end 85.75 52) (width 1) (layer B.Cu) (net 8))
 (segment (start 84.5 48.75) (end 85.75 50) (width 1) (layer B.Cu) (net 8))
 (segment (start 69.25 54.25) (end 68.25 53.25) (width 1) (layer B.Cu) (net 8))
 (segment (start 76.5 54.25) (end 69.25 54.25) (width 1) (layer B.Cu) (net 8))
 (segment (start 78.25 56) (end 76.5 54.25) (width 1) (layer B.Cu) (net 8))
 (segment (start 78.25 75.07) (end 78.25 56) (width 1) (layer B.Cu) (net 8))
 (segment (start 68.25 49) (end 68 48.75) (width 1) (layer B.Cu) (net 8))
 (segment (start 78.34 75.16) (end 78.25 75.07) (width 1) (layer B.Cu) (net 8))
 (segment (start 68 48.75) (end 84.5 48.75) (width 1) (layer B.Cu) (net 8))
 (segment (start 68.25 53.25) (end 68.25 49) (width 1) (layer B.Cu) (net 8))
 (segment (start 61.75 48.75) (end 68 48.75) (width 1) (layer B.Cu) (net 8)))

